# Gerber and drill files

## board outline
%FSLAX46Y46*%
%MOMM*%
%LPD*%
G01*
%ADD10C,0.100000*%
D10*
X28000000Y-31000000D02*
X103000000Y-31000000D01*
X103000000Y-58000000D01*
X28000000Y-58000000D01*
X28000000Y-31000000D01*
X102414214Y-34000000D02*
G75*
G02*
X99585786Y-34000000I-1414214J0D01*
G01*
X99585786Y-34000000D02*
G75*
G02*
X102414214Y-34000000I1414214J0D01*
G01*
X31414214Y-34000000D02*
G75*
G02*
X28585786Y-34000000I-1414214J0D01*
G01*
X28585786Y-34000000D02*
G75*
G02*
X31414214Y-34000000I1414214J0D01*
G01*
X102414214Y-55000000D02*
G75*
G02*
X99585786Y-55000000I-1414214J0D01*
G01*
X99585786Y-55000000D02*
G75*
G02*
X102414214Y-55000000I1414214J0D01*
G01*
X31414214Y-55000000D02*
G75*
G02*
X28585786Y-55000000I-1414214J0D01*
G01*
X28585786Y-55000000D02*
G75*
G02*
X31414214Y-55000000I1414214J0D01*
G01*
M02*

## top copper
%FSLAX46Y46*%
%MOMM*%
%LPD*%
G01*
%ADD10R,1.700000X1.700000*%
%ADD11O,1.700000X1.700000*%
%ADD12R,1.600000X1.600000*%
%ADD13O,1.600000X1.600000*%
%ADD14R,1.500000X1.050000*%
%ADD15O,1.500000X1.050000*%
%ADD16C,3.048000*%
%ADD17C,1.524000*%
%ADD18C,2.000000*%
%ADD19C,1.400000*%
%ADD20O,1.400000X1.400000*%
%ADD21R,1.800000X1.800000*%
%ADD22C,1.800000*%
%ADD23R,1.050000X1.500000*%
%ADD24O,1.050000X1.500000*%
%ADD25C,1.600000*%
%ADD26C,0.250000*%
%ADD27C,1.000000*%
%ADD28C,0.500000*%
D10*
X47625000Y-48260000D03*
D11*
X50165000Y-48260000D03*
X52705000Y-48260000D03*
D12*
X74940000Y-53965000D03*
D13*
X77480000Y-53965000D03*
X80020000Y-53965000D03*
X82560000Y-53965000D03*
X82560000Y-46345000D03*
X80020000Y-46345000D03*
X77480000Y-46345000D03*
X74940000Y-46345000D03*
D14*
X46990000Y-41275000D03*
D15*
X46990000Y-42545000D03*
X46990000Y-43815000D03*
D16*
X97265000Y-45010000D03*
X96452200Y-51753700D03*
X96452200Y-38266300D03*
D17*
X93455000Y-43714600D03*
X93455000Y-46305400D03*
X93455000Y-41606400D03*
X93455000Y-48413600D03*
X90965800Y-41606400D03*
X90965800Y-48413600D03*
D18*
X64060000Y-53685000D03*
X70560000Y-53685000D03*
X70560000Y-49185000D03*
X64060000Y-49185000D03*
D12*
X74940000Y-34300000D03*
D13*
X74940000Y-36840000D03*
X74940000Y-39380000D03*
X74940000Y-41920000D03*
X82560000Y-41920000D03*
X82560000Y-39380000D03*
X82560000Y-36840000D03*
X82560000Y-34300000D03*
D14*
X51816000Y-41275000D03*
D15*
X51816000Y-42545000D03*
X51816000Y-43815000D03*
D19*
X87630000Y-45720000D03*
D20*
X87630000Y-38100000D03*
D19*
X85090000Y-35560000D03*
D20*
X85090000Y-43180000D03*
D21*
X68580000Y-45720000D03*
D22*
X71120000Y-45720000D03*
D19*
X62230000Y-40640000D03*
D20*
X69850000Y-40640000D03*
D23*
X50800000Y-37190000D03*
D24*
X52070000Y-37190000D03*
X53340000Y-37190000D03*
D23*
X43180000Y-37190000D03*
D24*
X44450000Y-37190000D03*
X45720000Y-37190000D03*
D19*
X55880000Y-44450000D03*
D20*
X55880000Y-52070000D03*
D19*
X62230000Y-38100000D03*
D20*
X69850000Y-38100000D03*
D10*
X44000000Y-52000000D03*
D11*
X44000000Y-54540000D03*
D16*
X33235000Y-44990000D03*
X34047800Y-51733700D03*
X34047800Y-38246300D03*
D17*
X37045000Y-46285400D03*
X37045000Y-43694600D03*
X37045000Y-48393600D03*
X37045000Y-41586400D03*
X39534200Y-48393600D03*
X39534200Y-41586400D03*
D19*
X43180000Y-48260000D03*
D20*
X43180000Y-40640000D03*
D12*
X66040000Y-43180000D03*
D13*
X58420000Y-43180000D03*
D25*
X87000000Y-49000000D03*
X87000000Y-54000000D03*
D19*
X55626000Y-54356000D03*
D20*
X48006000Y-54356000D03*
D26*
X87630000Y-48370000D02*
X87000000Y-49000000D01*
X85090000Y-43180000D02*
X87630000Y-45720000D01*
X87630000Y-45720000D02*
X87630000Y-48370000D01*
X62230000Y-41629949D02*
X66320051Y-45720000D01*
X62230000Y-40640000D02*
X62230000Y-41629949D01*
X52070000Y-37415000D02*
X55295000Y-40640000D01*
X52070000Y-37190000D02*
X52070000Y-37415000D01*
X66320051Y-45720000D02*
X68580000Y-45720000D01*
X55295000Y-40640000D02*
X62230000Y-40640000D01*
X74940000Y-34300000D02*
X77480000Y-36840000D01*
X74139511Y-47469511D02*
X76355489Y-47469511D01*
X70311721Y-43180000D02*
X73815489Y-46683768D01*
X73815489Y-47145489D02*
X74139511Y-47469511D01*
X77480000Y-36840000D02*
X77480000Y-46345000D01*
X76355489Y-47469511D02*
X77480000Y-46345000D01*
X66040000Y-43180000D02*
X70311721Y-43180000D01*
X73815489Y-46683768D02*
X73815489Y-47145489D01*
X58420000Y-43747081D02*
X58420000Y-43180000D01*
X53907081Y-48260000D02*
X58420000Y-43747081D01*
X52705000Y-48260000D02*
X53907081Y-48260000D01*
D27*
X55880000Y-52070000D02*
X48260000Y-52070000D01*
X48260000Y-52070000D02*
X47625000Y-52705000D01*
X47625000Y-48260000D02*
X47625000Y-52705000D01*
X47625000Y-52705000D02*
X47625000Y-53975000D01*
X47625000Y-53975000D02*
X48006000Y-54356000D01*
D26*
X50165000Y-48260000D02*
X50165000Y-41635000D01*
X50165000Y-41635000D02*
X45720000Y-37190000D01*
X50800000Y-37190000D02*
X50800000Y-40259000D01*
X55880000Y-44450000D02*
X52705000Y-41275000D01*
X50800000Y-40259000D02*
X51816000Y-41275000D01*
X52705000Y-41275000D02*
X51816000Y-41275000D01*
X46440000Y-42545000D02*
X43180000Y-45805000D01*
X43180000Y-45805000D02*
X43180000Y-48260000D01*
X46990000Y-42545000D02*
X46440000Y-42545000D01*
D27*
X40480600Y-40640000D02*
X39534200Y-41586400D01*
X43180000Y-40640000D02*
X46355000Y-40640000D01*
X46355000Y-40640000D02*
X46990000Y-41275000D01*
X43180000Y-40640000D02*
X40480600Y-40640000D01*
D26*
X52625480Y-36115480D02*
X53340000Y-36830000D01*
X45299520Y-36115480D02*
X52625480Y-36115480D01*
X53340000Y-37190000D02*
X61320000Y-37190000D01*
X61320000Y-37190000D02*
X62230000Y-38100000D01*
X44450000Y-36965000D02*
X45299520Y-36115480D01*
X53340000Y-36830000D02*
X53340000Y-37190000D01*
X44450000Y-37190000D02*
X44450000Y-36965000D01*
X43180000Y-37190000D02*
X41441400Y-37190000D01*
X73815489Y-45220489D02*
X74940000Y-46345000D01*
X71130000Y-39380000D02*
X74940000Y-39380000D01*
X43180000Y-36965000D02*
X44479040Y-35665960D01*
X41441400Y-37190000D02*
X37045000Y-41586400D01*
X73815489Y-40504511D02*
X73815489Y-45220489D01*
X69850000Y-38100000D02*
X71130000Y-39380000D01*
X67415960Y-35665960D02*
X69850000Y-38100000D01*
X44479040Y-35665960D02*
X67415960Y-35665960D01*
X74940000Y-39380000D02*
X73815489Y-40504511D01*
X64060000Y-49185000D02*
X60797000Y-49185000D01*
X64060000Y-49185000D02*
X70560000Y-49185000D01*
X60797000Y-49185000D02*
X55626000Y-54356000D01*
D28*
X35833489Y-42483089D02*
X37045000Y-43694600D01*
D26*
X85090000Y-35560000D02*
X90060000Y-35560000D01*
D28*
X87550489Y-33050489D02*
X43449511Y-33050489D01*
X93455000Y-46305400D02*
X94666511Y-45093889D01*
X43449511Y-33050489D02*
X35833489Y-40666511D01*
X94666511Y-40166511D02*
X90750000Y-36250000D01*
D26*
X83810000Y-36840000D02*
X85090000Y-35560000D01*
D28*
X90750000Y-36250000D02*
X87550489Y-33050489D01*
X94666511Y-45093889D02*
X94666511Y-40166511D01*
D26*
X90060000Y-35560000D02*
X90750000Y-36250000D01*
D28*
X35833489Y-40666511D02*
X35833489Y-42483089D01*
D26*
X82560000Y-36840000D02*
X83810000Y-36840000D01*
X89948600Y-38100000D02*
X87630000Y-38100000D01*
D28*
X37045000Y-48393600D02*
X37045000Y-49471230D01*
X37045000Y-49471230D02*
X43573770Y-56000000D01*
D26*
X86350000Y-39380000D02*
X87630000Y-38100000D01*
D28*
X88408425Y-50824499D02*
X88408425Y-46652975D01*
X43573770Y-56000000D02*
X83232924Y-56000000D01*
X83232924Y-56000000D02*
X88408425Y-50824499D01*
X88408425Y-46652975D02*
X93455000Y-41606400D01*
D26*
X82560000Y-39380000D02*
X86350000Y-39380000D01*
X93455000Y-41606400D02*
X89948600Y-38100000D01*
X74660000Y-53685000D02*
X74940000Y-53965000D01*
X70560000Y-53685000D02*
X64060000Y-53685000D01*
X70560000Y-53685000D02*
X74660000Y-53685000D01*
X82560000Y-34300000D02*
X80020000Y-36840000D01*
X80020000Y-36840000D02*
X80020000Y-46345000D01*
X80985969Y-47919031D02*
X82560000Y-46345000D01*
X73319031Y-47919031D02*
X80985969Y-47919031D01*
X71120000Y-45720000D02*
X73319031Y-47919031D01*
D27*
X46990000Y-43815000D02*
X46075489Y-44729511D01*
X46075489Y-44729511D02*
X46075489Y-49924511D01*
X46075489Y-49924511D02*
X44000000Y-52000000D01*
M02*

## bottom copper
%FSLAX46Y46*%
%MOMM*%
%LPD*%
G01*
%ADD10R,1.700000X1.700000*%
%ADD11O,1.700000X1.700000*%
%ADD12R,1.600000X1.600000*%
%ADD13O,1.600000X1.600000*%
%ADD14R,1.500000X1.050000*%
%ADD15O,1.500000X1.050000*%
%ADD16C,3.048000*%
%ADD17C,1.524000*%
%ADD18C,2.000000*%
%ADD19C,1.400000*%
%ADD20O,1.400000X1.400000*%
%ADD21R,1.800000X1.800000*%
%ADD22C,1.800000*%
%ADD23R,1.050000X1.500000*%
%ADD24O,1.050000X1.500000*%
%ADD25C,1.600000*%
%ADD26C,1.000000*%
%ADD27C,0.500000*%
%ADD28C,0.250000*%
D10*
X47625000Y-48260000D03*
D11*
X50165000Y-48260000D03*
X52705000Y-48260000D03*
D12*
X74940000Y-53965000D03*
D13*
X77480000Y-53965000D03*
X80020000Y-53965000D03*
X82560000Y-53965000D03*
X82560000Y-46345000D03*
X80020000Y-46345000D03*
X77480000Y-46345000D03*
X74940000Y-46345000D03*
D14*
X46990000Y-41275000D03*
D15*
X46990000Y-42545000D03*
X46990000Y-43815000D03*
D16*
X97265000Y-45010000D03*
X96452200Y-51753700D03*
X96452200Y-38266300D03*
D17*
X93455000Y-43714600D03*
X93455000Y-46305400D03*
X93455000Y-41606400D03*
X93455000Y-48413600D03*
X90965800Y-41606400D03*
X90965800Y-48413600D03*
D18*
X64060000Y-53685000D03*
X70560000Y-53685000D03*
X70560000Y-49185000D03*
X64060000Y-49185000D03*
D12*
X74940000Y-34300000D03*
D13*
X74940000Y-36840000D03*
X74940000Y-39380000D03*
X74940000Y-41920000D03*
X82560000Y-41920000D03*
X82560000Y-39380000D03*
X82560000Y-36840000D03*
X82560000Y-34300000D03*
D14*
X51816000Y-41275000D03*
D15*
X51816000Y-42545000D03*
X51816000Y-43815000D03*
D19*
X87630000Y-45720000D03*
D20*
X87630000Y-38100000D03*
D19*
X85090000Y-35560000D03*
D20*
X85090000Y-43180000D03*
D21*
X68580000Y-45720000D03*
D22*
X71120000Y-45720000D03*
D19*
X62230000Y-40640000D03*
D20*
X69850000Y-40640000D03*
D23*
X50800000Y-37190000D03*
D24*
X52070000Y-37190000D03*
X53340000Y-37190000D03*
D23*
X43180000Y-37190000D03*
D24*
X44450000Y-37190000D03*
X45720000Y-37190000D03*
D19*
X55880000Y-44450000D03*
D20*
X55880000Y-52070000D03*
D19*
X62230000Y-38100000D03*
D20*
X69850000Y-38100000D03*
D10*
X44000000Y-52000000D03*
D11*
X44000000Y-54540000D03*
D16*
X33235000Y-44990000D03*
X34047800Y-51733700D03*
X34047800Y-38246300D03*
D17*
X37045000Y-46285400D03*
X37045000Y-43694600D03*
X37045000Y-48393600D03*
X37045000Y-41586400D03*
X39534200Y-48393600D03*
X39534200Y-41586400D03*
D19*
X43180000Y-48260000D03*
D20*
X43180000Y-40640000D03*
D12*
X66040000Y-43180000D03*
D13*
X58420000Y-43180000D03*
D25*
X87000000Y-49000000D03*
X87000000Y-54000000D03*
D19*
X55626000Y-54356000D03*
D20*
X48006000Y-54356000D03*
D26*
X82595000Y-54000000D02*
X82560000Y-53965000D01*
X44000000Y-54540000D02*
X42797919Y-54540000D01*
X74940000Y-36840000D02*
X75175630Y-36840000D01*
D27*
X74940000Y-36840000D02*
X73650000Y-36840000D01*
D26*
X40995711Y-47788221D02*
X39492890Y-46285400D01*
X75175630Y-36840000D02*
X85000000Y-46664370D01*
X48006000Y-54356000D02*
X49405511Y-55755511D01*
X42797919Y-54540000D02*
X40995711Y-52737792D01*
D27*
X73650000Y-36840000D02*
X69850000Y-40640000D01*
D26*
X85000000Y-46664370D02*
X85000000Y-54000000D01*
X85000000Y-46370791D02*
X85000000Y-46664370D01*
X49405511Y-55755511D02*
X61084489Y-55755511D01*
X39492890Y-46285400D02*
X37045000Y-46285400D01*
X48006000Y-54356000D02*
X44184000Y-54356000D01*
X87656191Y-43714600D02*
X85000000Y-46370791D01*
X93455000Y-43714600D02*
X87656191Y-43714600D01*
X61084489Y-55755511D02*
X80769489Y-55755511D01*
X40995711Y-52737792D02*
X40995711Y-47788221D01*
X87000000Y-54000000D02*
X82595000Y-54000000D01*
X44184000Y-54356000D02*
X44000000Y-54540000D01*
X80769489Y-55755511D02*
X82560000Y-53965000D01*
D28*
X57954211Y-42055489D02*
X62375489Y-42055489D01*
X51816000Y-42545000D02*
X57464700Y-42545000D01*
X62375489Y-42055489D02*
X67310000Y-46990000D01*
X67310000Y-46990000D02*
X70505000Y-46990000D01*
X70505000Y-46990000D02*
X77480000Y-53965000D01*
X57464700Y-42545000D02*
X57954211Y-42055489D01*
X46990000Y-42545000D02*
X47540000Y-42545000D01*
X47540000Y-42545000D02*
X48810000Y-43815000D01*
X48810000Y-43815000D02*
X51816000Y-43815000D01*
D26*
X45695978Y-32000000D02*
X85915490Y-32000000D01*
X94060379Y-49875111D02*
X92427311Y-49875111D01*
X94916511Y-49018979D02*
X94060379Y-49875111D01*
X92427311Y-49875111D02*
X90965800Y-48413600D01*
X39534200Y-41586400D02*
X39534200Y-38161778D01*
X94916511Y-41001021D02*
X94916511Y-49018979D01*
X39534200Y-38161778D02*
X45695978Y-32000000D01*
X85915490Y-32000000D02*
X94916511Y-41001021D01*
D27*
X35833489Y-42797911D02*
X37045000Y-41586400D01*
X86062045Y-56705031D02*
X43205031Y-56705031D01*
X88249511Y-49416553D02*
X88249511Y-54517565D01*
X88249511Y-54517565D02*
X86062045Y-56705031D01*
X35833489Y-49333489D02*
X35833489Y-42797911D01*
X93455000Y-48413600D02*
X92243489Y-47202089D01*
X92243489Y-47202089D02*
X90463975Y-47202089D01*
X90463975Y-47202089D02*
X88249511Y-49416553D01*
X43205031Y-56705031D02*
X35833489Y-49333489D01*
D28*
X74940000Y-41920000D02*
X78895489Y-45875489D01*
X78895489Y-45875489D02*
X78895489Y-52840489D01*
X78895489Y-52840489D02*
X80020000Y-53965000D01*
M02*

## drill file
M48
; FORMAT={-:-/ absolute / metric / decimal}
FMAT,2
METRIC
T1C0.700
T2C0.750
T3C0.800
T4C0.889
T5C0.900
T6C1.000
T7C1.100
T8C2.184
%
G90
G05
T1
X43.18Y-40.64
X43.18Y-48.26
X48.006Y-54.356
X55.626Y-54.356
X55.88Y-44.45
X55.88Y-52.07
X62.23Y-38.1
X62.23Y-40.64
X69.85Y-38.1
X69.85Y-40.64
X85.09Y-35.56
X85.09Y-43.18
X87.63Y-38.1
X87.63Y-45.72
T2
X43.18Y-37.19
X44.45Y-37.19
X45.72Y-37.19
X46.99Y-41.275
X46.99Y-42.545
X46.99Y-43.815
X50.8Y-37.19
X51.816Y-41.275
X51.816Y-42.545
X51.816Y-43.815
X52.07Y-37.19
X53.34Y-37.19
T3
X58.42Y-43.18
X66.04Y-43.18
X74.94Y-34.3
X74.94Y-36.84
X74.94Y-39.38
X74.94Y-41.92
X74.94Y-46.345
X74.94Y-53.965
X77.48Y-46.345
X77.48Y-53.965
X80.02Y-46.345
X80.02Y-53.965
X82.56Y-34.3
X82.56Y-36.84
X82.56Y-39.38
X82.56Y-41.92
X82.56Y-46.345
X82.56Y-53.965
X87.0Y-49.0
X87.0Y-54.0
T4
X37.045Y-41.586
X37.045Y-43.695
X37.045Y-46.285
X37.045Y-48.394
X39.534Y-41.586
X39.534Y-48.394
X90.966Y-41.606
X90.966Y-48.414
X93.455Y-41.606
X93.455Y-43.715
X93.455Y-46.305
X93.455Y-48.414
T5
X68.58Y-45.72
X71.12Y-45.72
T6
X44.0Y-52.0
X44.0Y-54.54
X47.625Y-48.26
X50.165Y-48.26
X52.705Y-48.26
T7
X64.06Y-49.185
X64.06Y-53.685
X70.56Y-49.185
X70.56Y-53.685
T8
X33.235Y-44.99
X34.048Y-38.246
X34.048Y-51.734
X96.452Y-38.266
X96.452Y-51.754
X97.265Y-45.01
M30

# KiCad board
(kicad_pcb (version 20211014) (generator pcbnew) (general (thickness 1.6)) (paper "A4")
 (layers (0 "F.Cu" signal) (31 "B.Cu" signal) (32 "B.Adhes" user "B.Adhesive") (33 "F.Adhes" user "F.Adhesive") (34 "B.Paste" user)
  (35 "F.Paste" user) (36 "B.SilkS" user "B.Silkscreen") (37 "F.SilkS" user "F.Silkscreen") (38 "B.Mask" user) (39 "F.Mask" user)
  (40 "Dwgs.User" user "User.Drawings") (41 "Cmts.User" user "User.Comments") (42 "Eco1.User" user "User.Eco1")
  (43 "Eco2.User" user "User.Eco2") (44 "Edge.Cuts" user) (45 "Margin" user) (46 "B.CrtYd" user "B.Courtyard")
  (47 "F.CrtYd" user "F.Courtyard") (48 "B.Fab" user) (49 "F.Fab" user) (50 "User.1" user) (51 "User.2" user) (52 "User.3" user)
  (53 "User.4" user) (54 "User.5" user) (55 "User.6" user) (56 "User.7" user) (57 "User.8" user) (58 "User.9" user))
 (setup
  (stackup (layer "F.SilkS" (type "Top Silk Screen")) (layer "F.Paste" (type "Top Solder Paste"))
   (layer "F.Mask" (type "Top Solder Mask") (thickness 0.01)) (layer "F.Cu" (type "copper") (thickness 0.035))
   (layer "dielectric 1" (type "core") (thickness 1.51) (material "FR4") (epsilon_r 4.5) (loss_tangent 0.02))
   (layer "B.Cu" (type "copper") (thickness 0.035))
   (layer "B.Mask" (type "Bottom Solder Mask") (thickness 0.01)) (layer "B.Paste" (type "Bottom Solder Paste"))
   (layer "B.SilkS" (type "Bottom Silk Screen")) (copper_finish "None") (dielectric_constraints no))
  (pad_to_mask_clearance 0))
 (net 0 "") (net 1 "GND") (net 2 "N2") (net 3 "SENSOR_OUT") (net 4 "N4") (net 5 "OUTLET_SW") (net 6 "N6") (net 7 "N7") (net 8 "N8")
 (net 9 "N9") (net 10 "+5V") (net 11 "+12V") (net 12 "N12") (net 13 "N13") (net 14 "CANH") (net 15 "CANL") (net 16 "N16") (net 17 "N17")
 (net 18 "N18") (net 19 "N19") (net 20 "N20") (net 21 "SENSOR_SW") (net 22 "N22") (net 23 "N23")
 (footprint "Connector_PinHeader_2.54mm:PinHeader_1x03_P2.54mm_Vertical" (layer "F.Cu") (at 47.625 48.26 90)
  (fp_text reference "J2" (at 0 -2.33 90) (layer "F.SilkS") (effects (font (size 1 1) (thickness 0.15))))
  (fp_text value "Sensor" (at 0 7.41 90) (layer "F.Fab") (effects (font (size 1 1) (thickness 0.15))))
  (pad "1" thru_hole rect (at 0 0 90) (size 1.7 1.7) (drill 1) (layers *.Cu *.Mask) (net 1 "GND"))
  (pad "2" thru_hole oval (at 0 2.54 90) (size 1.7 1.7) (drill 1) (layers *.Cu *.Mask) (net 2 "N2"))
  (pad "3" thru_hole oval (at 0 5.08 90) (size 1.7 1.7) (drill 1) (layers *.Cu *.Mask) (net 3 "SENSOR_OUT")))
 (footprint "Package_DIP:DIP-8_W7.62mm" (layer "F.Cu") (at 74.94 53.965 90)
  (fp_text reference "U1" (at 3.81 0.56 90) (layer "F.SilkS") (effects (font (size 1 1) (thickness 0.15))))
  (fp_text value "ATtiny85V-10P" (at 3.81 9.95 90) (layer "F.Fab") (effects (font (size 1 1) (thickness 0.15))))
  (pad "1" thru_hole rect (at 0 0 90) (size 1.6 1.6) (drill 0.8) (layers *.Cu *.Mask) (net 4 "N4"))
  (pad "2" thru_hole oval (at 0 2.54 90) (size 1.6 1.6) (drill 0.8) (layers *.Cu *.Mask) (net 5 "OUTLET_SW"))
  (pad "3" thru_hole oval (at 0 5.08 90) (size 1.6 1.6) (drill 0.8) (layers *.Cu *.Mask) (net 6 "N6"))
  (pad "4" thru_hole oval (at 0 7.62 90) (size 1.6 1.6) (drill 0.8) (layers *.Cu *.Mask) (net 1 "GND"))
  (pad "5" thru_hole oval (at 7.62 7.62 90) (size 1.6 1.6) (drill 0.8) (layers *.Cu *.Mask) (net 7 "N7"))
  (pad "6" thru_hole oval (at 7.62 5.08 90) (size 1.6 1.6) (drill 0.8) (layers *.Cu *.Mask) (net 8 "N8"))
  (pad "7" thru_hole oval (at 7.62 2.54 90) (size 1.6 1.6) (drill 0.8) (layers *.Cu *.Mask) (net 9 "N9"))
  (pad "8" thru_hole oval (at 7.62 0 90) (size 1.6 1.6) (drill 0.8) (layers *.Cu *.Mask) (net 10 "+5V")))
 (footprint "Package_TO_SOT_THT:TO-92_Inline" (layer "F.Cu") (at 46.99 41.275 -90)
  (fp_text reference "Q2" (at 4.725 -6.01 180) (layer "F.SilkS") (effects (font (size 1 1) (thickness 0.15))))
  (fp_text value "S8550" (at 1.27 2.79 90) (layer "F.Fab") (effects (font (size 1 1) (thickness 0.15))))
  (pad "1" thru_hole rect (at 0 0 270) (size 1.05 1.5) (drill 0.75) (layers *.Cu *.Mask) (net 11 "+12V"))
  (pad "2" thru_hole oval (at 1.27 0 270) (size 1.05 1.5) (drill 0.75) (layers *.Cu *.Mask) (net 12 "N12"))
  (pad "3" thru_hole oval (at 2.54 0 270) (size 1.05 1.5) (drill 0.75) (layers *.Cu *.Mask) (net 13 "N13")))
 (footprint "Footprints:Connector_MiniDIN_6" (layer "F.Cu") (at 97.265 45.01 -90)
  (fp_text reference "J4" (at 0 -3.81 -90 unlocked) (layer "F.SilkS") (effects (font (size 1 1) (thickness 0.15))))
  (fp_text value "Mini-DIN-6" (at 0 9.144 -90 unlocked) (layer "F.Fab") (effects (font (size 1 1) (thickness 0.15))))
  (pad "" thru_hole circle (at 0 0 270) (size 3.048 3.048) (drill 2.1844) (layers *.Cu *.Mask))
  (pad "" thru_hole circle (at 6.7437 0.8128 270) (size 3.048 3.048) (drill 2.1844) (layers *.Cu *.Mask))
  (pad "" thru_hole circle (at -6.7437 0.8128 270) (size 3.048 3.048) (drill 2.1844) (layers *.Cu *.Mask))
  (pad "1" thru_hole circle (at -1.2954 3.81 270) (size 1.524 1.524) (drill 0.889) (layers *.Cu *.Mask) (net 1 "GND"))
  (pad "2" thru_hole circle (at 1.2954 3.81 270) (size 1.524 1.524) (drill 0.889) (layers *.Cu *.Mask) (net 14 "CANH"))
  (pad "3" thru_hole circle (at -3.4036 3.81 270) (size 1.524 1.524) (drill 0.889) (layers *.Cu *.Mask) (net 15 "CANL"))
  (pad "4" thru_hole circle (at 3.4036 3.81 270) (size 1.524 1.524) (drill 0.889) (layers *.Cu *.Mask) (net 10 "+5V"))
  (pad "5" thru_hole circle (at -3.4036 6.2992 270) (size 1.524 1.524) (drill 0.889) (layers *.Cu *.Mask) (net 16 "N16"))
  (pad "6" thru_hole circle (at 3.4036 6.2992 270) (size 1.524 1.524) (drill 0.889) (layers *.Cu *.Mask) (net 11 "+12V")))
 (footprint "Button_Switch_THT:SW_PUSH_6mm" (layer "F.Cu") (at 70.56 53.685 180)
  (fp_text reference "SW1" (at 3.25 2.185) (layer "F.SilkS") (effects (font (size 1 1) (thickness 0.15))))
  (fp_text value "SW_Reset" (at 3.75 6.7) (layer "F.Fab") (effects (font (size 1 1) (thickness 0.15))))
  (pad "1" thru_hole circle (at 6.5 0 270) (size 2 2) (drill 1.1) (layers *.Cu *.Mask) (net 4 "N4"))
  (pad "1" thru_hole circle (at 0 0 270) (size 2 2) (drill 1.1) (layers *.Cu *.Mask) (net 4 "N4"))
  (pad "2" thru_hole circle (at 0 4.5 270) (size 2 2) (drill 1.1) (layers *.Cu *.Mask) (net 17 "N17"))
  (pad "2" thru_hole circle (at 6.5 4.5 270) (size 2 2) (drill 1.1) (layers *.Cu *.Mask) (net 17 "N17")))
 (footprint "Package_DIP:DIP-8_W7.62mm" (layer "F.Cu") (at 74.94 34.3)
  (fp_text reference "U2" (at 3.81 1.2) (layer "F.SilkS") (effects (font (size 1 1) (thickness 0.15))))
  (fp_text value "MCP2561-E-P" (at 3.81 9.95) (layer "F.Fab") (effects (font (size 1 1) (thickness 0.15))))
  (pad "1" thru_hole rect (at 0 0) (size 1.6 1.6) (drill 0.8) (layers *.Cu *.Mask) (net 9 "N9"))
  (pad "2" thru_hole oval (at 0 2.54) (size 1.6 1.6) (drill 0.8) (layers *.Cu *.Mask) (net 1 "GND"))
  (pad "3" thru_hole oval (at 0 5.08) (size 1.6 1.6) (drill 0.8) (layers *.Cu *.Mask) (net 10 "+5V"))
  (pad "4" thru_hole oval (at 0 7.62) (size 1.6 1.6) (drill 0.8) (layers *.Cu *.Mask) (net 6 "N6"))
  (pad "5" thru_hole oval (at 7.62 7.62) (size 1.6 1.6) (drill 0.8) (layers *.Cu *.Mask) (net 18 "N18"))
  (pad "6" thru_hole oval (at 7.62 5.08) (size 1.6 1.6) (drill 0.8) (layers *.Cu *.Mask) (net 15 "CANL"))
  (pad "7" thru_hole oval (at 7.62 2.54) (size 1.6 1.6) (drill 0.8) (layers *.Cu *.Mask) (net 14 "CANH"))
  (pad "8" thru_hole oval (at 7.62 0) (size 1.6 1.6) (drill 0.8) (layers *.Cu *.Mask) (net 8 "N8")))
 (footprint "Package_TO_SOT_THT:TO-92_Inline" (layer "F.Cu") (at 51.816 41.275 -90)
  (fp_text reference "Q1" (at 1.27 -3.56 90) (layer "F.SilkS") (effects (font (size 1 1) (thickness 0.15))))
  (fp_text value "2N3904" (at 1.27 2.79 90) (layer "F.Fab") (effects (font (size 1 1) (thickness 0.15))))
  (pad "1" thru_hole rect (at 0 0 270) (size 1.05 1.5) (drill 0.75) (layers *.Cu *.Mask) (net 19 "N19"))
  (pad "2" thru_hole oval (at 1.27 0 270) (size 1.05 1.5) (drill 0.75) (layers *.Cu *.Mask) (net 5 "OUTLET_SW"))
  (pad "3" thru_hole oval (at 2.54 0 270) (size 1.05 1.5) (drill 0.75) (layers *.Cu *.Mask) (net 12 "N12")))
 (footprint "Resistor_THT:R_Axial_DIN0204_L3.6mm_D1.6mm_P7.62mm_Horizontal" (layer "F.Cu") (at 87.63 45.72 90)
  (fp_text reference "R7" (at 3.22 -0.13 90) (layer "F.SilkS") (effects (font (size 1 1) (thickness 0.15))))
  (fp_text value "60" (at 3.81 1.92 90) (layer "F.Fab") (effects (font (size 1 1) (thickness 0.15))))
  (pad "1" thru_hole circle (at 0 0 90) (size 1.4 1.4) (drill 0.7) (layers *.Cu *.Mask) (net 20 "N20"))
  (pad "2" thru_hole oval (at 7.62 0 90) (size 1.4 1.4) (drill 0.7) (layers *.Cu *.Mask) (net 15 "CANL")))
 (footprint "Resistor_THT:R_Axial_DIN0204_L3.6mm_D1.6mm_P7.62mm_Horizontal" (layer "F.Cu") (at 85.09 35.56 -90)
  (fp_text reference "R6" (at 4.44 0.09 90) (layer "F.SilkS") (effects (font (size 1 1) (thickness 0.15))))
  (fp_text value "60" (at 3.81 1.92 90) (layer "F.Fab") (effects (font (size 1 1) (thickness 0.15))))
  (pad "1" thru_hole circle (at 0 0 270) (size 1.4 1.4) (drill 0.7) (layers *.Cu *.Mask) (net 14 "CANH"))
  (pad "2" thru_hole oval (at 7.62 0 270) (size 1.4 1.4) (drill 0.7) (layers *.Cu *.Mask) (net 20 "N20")))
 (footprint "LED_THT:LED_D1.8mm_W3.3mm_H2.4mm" (layer "F.Cu") (at 68.58 45.72)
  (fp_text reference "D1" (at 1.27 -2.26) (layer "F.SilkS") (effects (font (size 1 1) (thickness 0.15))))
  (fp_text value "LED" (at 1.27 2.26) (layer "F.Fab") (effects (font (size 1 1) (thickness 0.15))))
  (pad "1" thru_hole rect (at 0 0) (size 1.8 1.8) (drill 0.9) (layers *.Cu *.Mask) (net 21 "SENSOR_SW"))
  (pad "2" thru_hole circle (at 2.54 0) (size 1.8 1.8) (drill 0.9) (layers *.Cu *.Mask) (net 7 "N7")))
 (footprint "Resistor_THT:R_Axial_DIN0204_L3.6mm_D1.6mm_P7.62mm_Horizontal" (layer "F.Cu") (at 62.23 40.64)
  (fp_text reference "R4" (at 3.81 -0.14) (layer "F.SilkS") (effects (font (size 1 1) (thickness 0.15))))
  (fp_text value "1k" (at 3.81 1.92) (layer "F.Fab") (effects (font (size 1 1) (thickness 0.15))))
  (pad "1" thru_hole circle (at 0 0) (size 1.4 1.4) (drill 0.7) (layers *.Cu *.Mask) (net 21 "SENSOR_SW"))
  (pad "2" thru_hole oval (at 7.62 0) (size 1.4 1.4) (drill 0.7) (layers *.Cu *.Mask) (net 1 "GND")))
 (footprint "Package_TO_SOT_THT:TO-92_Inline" (layer "F.Cu") (at 50.8 37.19)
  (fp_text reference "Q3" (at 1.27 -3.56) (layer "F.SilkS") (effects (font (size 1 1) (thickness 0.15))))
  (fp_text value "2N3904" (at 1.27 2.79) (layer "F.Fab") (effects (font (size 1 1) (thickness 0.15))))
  (pad "1" thru_hole rect (at 0 0) (size 1.05 1.5) (drill 0.75) (layers *.Cu *.Mask) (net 19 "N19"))
  (pad "2" thru_hole oval (at 1.27 0) (size 1.05 1.5) (drill 0.75) (layers *.Cu *.Mask) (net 21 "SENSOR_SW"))
  (pad "3" thru_hole oval (at 2.54 0) (size 1.05 1.5) (drill 0.75) (layers *.Cu *.Mask) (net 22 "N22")))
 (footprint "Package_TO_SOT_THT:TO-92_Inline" (layer "F.Cu") (at 43.18 37.19)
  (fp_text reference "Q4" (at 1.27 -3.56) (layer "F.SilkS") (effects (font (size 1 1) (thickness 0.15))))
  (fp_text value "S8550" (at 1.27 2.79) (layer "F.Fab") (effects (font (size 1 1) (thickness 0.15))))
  (pad "1" thru_hole rect (at 0 0) (size 1.05 1.5) (drill 0.75) (layers *.Cu *.Mask) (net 10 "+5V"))
  (pad "2" thru_hole oval (at 1.27 0) (size 1.05 1.5) (drill 0.75) (layers *.Cu *.Mask) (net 22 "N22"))
  (pad "3" thru_hole oval (at 2.54 0) (size 1.05 1.5) (drill 0.75) (layers *.Cu *.Mask) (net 2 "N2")))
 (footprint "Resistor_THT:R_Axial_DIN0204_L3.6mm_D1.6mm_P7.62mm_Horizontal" (layer "F.Cu") (at 55.88 44.45 -90)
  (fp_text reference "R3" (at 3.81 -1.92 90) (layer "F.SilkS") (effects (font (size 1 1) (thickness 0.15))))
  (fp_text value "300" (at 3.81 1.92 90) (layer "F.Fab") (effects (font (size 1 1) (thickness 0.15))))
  (pad "1" thru_hole circle (at 0 0 270) (size 1.4 1.4) (drill 0.7) (layers *.Cu *.Mask) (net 19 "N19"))
  (pad "2" thru_hole oval (at 7.62 0 270) (size 1.4 1.4) (drill 0.7) (layers *.Cu *.Mask) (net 1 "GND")))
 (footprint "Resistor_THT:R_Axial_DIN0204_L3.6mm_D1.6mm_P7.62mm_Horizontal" (layer "F.Cu") (at 62.23 38.1)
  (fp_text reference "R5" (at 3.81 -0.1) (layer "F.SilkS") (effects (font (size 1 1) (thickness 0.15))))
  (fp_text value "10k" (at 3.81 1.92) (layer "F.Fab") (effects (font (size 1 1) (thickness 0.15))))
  (pad "1" thru_hole circle (at 0 0) (size 1.4 1.4) (drill 0.7) (layers *.Cu *.Mask) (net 22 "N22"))
  (pad "2" thru_hole oval (at 7.62 0) (size 1.4 1.4) (drill 0.7) (layers *.Cu *.Mask) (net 10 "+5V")))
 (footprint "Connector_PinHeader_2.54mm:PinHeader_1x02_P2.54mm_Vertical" (layer "F.Cu") (at 44 52)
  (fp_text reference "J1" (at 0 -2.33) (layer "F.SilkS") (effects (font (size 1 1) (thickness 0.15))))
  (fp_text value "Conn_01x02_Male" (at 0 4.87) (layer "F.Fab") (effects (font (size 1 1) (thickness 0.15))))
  (pad "1" thru_hole rect (at 0 0) (size 1.7 1.7) (drill 1) (layers *.Cu *.Mask) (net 13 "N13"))
  (pad "2" thru_hole oval (at 0 2.54) (size 1.7 1.7) (drill 1) (layers *.Cu *.Mask) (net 1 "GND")))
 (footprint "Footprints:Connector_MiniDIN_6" (layer "F.Cu") (at 33.235 44.99 90)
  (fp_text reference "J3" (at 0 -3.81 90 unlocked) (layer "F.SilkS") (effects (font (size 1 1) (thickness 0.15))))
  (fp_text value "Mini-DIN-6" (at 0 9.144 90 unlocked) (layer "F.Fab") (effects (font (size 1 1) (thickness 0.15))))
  (pad "" thru_hole circle (at 0 0 90) (size 3.048 3.048) (drill 2.1844) (layers *.Cu *.Mask))
  (pad "" thru_hole circle (at -6.7437 0.8128 90) (size 3.048 3.048) (drill 2.1844) (layers *.Cu *.Mask))
  (pad "" thru_hole circle (at 6.7437 0.8128 90) (size 3.048 3.048) (drill 2.1844) (layers *.Cu *.Mask))
  (pad "1" thru_hole circle (at -1.2954 3.81 90) (size 1.524 1.524) (drill 0.889) (layers *.Cu *.Mask) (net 1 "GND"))
  (pad "2" thru_hole circle (at 1.2954 3.81 90) (size 1.524 1.524) (drill 0.889) (layers *.Cu *.Mask) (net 14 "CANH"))
  (pad "3" thru_hole circle (at -3.4036 3.81 90) (size 1.524 1.524) (drill 0.889) (layers *.Cu *.Mask) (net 15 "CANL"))
  (pad "4" thru_hole circle (at 3.4036 3.81 90) (size 1.524 1.524) (drill 0.889) (layers *.Cu *.Mask) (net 10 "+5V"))
  (pad "5" thru_hole circle (at -3.4036 6.2992 90) (size 1.524 1.524) (drill 0.889) (layers *.Cu *.Mask) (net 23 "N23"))
  (pad "6" thru_hole circle (at 3.4036 6.2992 90) (size 1.524 1.524) (drill 0.889) (layers *.Cu *.Mask) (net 11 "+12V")))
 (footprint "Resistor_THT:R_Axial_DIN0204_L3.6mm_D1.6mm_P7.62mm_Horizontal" (layer "F.Cu") (at 43.18 48.26 90)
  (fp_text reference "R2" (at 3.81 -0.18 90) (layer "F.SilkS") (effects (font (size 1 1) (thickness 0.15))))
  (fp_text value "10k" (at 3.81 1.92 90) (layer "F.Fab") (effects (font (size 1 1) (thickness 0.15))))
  (pad "1" thru_hole circle (at 0 0 90) (size 1.4 1.4) (drill 0.7) (layers *.Cu *.Mask) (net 12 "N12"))
  (pad "2" thru_hole oval (at 7.62 0 90) (size 1.4 1.4) (drill 0.7) (layers *.Cu *.Mask) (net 11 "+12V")))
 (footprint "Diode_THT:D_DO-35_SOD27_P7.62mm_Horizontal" (layer "F.Cu") (at 66.04 43.18 180)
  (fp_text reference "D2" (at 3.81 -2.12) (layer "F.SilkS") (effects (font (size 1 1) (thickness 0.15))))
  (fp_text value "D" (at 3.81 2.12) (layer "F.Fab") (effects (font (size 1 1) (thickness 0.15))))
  (pad "1" thru_hole rect (at 0 0 180) (size 1.6 1.6) (drill 0.8) (layers *.Cu *.Mask) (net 9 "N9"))
  (pad "2" thru_hole oval (at 7.62 0 180) (size 1.6 1.6) (drill 0.8) (layers *.Cu *.Mask) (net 3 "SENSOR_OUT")))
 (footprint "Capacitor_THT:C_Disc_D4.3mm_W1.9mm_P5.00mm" (layer "F.Cu") (at 87 49 -90)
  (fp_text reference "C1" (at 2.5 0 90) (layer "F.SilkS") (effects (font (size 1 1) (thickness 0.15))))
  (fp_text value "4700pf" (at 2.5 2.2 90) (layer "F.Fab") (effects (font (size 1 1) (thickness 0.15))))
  (pad "1" thru_hole circle (at 0 0 270) (size 1.6 1.6) (drill 0.8) (layers *.Cu *.Mask) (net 20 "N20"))
  (pad "2" thru_hole circle (at 5 0 270) (size 1.6 1.6) (drill 0.8) (layers *.Cu *.Mask) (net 1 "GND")))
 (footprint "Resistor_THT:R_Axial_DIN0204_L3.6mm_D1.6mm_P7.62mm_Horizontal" (layer "F.Cu") (at 55.626 54.356 180)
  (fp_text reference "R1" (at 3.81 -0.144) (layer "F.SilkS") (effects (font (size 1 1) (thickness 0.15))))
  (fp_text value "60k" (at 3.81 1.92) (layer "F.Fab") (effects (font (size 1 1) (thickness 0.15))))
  (pad "1" thru_hole circle (at 0 0 180) (size 1.4 1.4) (drill 0.7) (layers *.Cu *.Mask) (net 17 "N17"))
  (pad "2" thru_hole oval (at 7.62 0 180) (size 1.4 1.4) (drill 0.7) (layers *.Cu *.Mask) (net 1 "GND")))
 (gr_rect (start 28 31) (end 103 58) (layer "Edge.Cuts") (width 0.1) (fill none))
 (gr_circle (center 101 34) (end 102 35) (layer "Edge.Cuts") (width 0.1) (fill none))
 (gr_circle (center 30 34) (end 31 35) (layer "Edge.Cuts") (width 0.1) (fill none))
 (gr_circle (center 101 55) (end 102 56) (layer "Edge.Cuts") (width 0.1) (fill none))
 (gr_circle (center 30 55) (end 31 56) (layer "Edge.Cuts") (width 0.1) (fill none))
 (segment (start 87.63 48.37) (end 87 49) (width 0.25) (layer "F.Cu") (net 20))
 (segment (start 85.09 43.18) (end 87.63 45.72) (width 0.25) (layer "F.Cu") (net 20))
 (segment (start 87.63 45.72) (end 87.63 48.37) (width 0.25) (layer "F.Cu") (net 20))
 (segment (start 62.23 41.629949) (end 66.320051 45.72) (width 0.25) (layer "F.Cu") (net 21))
 (segment (start 62.23 40.64) (end 62.23 41.629949) (width 0.25) (layer "F.Cu") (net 21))
 (segment (start 52.07 37.415) (end 55.295 40.64) (width 0.25) (layer "F.Cu") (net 21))
 (segment (start 52.07 37.19) (end 52.07 37.415) (width 0.25) (layer "F.Cu") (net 21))
 (segment (start 66.320051 45.72) (end 68.58 45.72) (width 0.25) (layer "F.Cu") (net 21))
 (segment (start 55.295 40.64) (end 62.23 40.64) (width 0.25) (layer "F.Cu") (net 21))
 (segment (start 74.94 34.3) (end 77.48 36.84) (width 0.25) (layer "F.Cu") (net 9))
 (segment (start 74.139511 47.469511) (end 76.355489 47.469511) (width 0.25) (layer "F.Cu") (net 9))
 (segment (start 70.311721 43.18) (end 73.815489 46.683768) (width 0.25) (layer "F.Cu") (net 9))
 (segment (start 73.815489 47.145489) (end 74.139511 47.469511) (width 0.25) (layer "F.Cu") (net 9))
 (segment (start 77.48 36.84) (end 77.48 46.345) (width 0.25) (layer "F.Cu") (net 9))
 (segment (start 76.355489 47.469511) (end 77.48 46.345) (width 0.25) (layer "F.Cu") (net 9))
 (segment (start 66.04 43.18) (end 70.311721 43.18) (width 0.25) (layer "F.Cu") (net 9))
 (segment (start 73.815489 46.683768) (end 73.815489 47.145489) (width 0.25) (layer "F.Cu") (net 9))
 (segment (start 58.42 43.747081) (end 58.42 43.18) (width 0.25) (layer "F.Cu") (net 3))
 (segment (start 53.907081 48.26) (end 58.42 43.747081) (width 0.25) (layer "F.Cu") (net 3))
 (segment (start 52.705 48.26) (end 53.907081 48.26) (width 0.25) (layer "F.Cu") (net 3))
 (segment (start 55.88 52.07) (end 48.26 52.07) (width 1) (layer "F.Cu") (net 1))
 (segment (start 48.26 52.07) (end 47.625 52.705) (width 1) (layer "F.Cu") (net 1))
 (segment (start 47.625 48.26) (end 47.625 52.705) (width 1) (layer "F.Cu") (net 1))
 (segment (start 47.625 52.705) (end 47.625 53.975) (width 1) (layer "F.Cu") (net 1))
 (segment (start 47.625 53.975) (end 48.006 54.356) (width 1) (layer "F.Cu") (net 1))
 (segment (start 82.595 54) (end 82.56 53.965) (width 1) (layer "B.Cu") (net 1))
 (segment (start 44 54.54) (end 42.797919 54.54) (width 1) (layer "B.Cu") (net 1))
 (segment (start 74.94 36.84) (end 75.17563 36.84) (width 1) (layer "B.Cu") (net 1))
 (segment (start 74.94 36.84) (end 73.65 36.84) (width 0.5) (layer "B.Cu") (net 1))
 (segment (start 40.995711 47.788221) (end 39.49289 46.2854) (width 1) (layer "B.Cu") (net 1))
 (segment (start 75.17563 36.84) (end 85 46.66437) (width 1) (layer "B.Cu") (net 1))
 (segment (start 48.006 54.356) (end 49.405511 55.755511) (width 1) (layer "B.Cu") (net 1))
 (segment (start 42.797919 54.54) (end 40.995711 52.737792) (width 1) (layer "B.Cu") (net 1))
 (segment (start 73.65 36.84) (end 69.85 40.64) (width 0.5) (layer "B.Cu") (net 1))
 (segment (start 85 46.66437) (end 85 54) (width 1) (layer "B.Cu") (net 1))
 (segment (start 85 46.370791) (end 85 46.66437) (width 1) (layer "B.Cu") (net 1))
 (segment (start 49.405511 55.755511) (end 61.084489 55.755511) (width 1) (layer "B.Cu") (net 1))
 (segment (start 39.49289 46.2854) (end 37.045 46.2854) (width 1) (layer "B.Cu") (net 1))
 (segment (start 48.006 54.356) (end 44.184 54.356) (width 1) (layer "B.Cu") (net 1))
 (segment (start 87.656191 43.7146) (end 85 46.370791) (width 1) (layer "B.Cu") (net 1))
 (segment (start 93.455 43.7146) (end 87.656191 43.7146) (width 1) (layer "B.Cu") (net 1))
 (segment (start 61.084489 55.755511) (end 80.769489 55.755511) (width 1) (layer "B.Cu") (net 1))
 (segment (start 40.995711 52.737792) (end 40.995711 47.788221) (width 1) (layer "B.Cu") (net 1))
 (segment (start 87 54) (end 82.595 54) (width 1) (layer "B.Cu") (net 1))
 (segment (start 44.184 54.356) (end 44 54.54) (width 1) (layer "B.Cu") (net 1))
 (segment (start 80.769489 55.755511) (end 82.56 53.965) (width 1) (layer "B.Cu") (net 1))
 (segment (start 50.165 48.26) (end 50.165 41.635) (width 0.25) (layer "F.Cu") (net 2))
 (segment (start 50.165 41.635) (end 45.72 37.19) (width 0.25) (layer "F.Cu") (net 2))
 (segment (start 50.8 37.19) (end 50.8 40.259) (width 0.25) (layer "F.Cu") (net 19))
 (segment (start 55.88 44.45) (end 52.705 41.275) (width 0.25) (layer "F.Cu") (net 19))
 (segment (start 50.8 40.259) (end 51.816 41.275) (width 0.25) (layer "F.Cu") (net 19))
 (segment (start 52.705 41.275) (end 51.816 41.275) (width 0.25) (layer "F.Cu") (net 19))
 (segment (start 57.954211 42.055489) (end 62.375489 42.055489) (width 0.25) (layer "B.Cu") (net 5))
 (segment (start 51.816 42.545) (end 57.4647 42.545) (width 0.25) (layer "B.Cu") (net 5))
 (segment (start 62.375489 42.055489) (end 67.31 46.99) (width 0.25) (layer "B.Cu") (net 5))
 (segment (start 67.31 46.99) (end 70.505 46.99) (width 0.25) (layer "B.Cu") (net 5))
 (segment (start 70.505 46.99) (end 77.48 53.965) (width 0.25) (layer "B.Cu") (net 5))
 (segment (start 57.4647 42.545) (end 57.954211 42.055489) (width 0.25) (layer "B.Cu") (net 5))
 (segment (start 46.44 42.545) (end 43.18 45.805) (width 0.25) (layer "F.Cu") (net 12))
 (segment (start 43.18 45.805) (end 43.18 48.26) (width 0.25) (layer "F.Cu") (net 12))
 (segment (start 46.99 42.545) (end 46.44 42.545) (width 0.25) (layer "F.Cu") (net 12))
 (segment (start 46.99 42.545) (end 47.54 42.545) (width 0.25) (layer "B.Cu") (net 12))
 (segment (start 47.54 42.545) (end 48.81 43.815) (width 0.25) (layer "B.Cu") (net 12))
 (segment (start 48.81 43.815) (end 51.816 43.815) (width 0.25) (layer "B.Cu") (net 12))
 (segment (start 40.4806 40.64) (end 39.5342 41.5864) (width 1) (layer "F.Cu") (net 11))
 (segment (start 43.18 40.64) (end 46.355 40.64) (width 1) (layer "F.Cu") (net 11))
 (segment (start 46.355 40.64) (end 46.99 41.275) (width 1) (layer "F.Cu") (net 11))
 (segment (start 43.18 40.64) (end 40.4806 40.64) (width 1) (layer "F.Cu") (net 11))
 (segment (start 45.695978 32) (end 85.91549 32) (width 1) (layer "B.Cu") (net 11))
 (segment (start 94.060379 49.875111) (end 92.427311 49.875111) (width 1) (layer "B.Cu") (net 11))
 (segment (start 94.916511 49.018979) (end 94.060379 49.875111) (width 1) (layer "B.Cu") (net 11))
 (segment (start 92.427311 49.875111) (end 90.9658 48.4136) (width 1) (layer "B.Cu") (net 11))
 (segment (start 39.5342 41.5864) (end 39.5342 38.161778) (width 1) (layer "B.Cu") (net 11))
 (segment (start 94.916511 41.001021) (end 94.916511 49.018979) (width 1) (layer "B.Cu") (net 11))
 (segment (start 39.5342 38.161778) (end 45.695978 32) (width 1) (layer "B.Cu") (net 11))
 (segment (start 85.91549 32) (end 94.916511 41.001021) (width 1) (layer "B.Cu") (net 11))
 (segment (start 52.62548 36.11548) (end 53.34 36.83) (width 0.25) (layer "F.Cu") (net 22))
 (segment (start 45.29952 36.11548) (end 52.62548 36.11548) (width 0.25) (layer "F.Cu") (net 22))
 (segment (start 53.34 37.19) (end 61.32 37.19) (width 0.25) (layer "F.Cu") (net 22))
 (segment (start 61.32 37.19) (end 62.23 38.1) (width 0.25) (layer "F.Cu") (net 22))
 (segment (start 44.45 36.965) (end 45.29952 36.11548) (width 0.25) (layer "F.Cu") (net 22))
 (segment (start 53.34 36.83) (end 53.34 37.19) (width 0.25) (layer "F.Cu") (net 22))
 (segment (start 44.45 37.19) (end 44.45 36.965) (width 0.25) (layer "F.Cu") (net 22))
 (segment (start 43.18 37.19) (end 41.4414 37.19) (width 0.25) (layer "F.Cu") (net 10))
 (segment (start 73.815489 45.220489) (end 74.94 46.345) (width 0.25) (layer "F.Cu") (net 10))
 (segment (start 71.13 39.38) (end 74.94 39.38) (width 0.25) (layer "F.Cu") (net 10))
 (segment (start 43.18 36.965) (end 44.47904 35.66596) (width 0.25) (layer "F.Cu") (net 10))
 (segment (start 41.4414 37.19) (end 37.045 41.5864) (width 0.25) (layer "F.Cu") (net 10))
 (segment (start 73.815489 40.504511) (end 73.815489 45.220489) (width 0.25) (layer "F.Cu") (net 10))
 (segment (start 69.85 38.1) (end 71.13 39.38) (width 0.25) (layer "F.Cu") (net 10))
 (segment (start 67.41596 35.66596) (end 69.85 38.1) (width 0.25) (layer "F.Cu") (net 10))
 (segment (start 44.47904 35.66596) (end 67.41596 35.66596) (width 0.25) (layer "F.Cu") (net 10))
 (segment (start 74.94 39.38) (end 73.815489 40.504511) (width 0.25) (layer "F.Cu") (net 10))
 (segment (start 35.833489 42.797911) (end 37.045 41.5864) (width 0.5) (layer "B.Cu") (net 10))
 (segment (start 86.062045 56.705031) (end 43.205031 56.705031) (width 0.5) (layer "B.Cu") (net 10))
 (segment (start 88.249511 49.416553) (end 88.249511 54.517565) (width 0.5) (layer "B.Cu") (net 10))
 (segment (start 88.249511 54.517565) (end 86.062045 56.705031) (width 0.5) (layer "B.Cu") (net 10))
 (segment (start 35.833489 49.333489) (end 35.833489 42.797911) (width 0.5) (layer "B.Cu") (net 10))
 (segment (start 93.455 48.4136) (end 92.243489 47.202089) (width 0.5) (layer "B.Cu") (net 10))
 (segment (start 92.243489 47.202089) (end 90.463975 47.202089) (width 0.5) (layer "B.Cu") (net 10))
 (segment (start 90.463975 47.202089) (end 88.249511 49.416553) (width 0.5) (layer "B.Cu") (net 10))
 (segment (start 43.205031 56.705031) (end 35.833489 49.333489) (width 0.5) (layer "B.Cu") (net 10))
 (segment (start 64.06 49.185) (end 60.797 49.185) (width 0.25) (layer "F.Cu") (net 17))
 (segment (start 64.06 49.185) (end 70.56 49.185) (width 0.25) (layer "F.Cu") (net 17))
 (segment (start 60.797 49.185) (end 55.626 54.356) (width 0.25) (layer "F.Cu") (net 17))
 (segment (start 35.833489 42.483089) (end 37.045 43.6946) (width 0.5) (layer "F.Cu") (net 14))
 (segment (start 85.09 35.56) (end 90.06 35.56) (width 0.25) (layer "F.Cu") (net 14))
 (segment (start 87.550489 33.050489) (end 43.449511 33.050489) (width 0.5) (layer "F.Cu") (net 14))
 (segment (start 93.455 46.3054) (end 94.666511 45.093889) (width 0.5) (layer "F.Cu") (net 14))
 (segment (start 43.449511 33.050489) (end 35.833489 40.666511) (width 0.5) (layer "F.Cu") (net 14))
 (segment (start 94.666511 40.166511) (end 90.75 36.25) (width 0.5) (layer "F.Cu") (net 14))
 (segment (start 83.81 36.84) (end 85.09 35.56) (width 0.25) (layer "F.Cu") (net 14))
 (segment (start 90.75 36.25) (end 87.550489 33.050489) (width 0.5) (layer "F.Cu") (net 14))
 (segment (start 94.666511 45.093889) (end 94.666511 40.166511) (width 0.5) (layer "F.Cu") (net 14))
 (segment (start 90.06 35.56) (end 90.75 36.25) (width 0.25) (layer "F.Cu") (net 14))
 (segment (start 35.833489 40.666511) (end 35.833489 42.483089) (width 0.5) (layer "F.Cu") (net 14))
 (segment (start 82.56 36.84) (end 83.81 36.84) (width 0.25) (layer "F.Cu") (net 14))
 (segment (start 89.9486 38.1) (end 87.63 38.1) (width 0.25) (layer "F.Cu") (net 15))
 (segment (start 37.045 48.3936) (end 37.045 49.47123) (width 0.5) (layer "F.Cu") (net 15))
 (segment (start 37.045 49.47123) (end 43.57377 56) (width 0.5) (layer "F.Cu") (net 15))
 (segment (start 86.35 39.38) (end 87.63 38.1) (width 0.25) (layer "F.Cu") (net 15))
 (segment (start 88.408425 50.824499) (end 88.408425 46.652975) (width 0.5) (layer "F.Cu") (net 15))
 (segment (start 43.57377 56) (end 83.232924 56) (width 0.5) (layer "F.Cu") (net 15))
 (segment (start 83.232924 56) (end 88.408425 50.824499) (width 0.5) (layer "F.Cu") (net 15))
 (segment (start 88.408425 46.652975) (end 93.455 41.6064) (width 0.5) (layer "F.Cu") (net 15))
 (segment (start 82.56 39.38) (end 86.35 39.38) (width 0.25) (layer "F.Cu") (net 15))
 (segment (start 93.455 41.6064) (end 89.9486 38.1) (width 0.25) (layer "F.Cu") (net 15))
 (segment (start 74.66 53.685) (end 74.94 53.965) (width 0.25) (layer "F.Cu") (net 4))
 (segment (start 70.56 53.685) (end 64.06 53.685) (width 0.25) (layer "F.Cu") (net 4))
 (segment (start 70.56 53.685) (end 74.66 53.685) (width 0.25) (layer "F.Cu") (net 4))
 (segment (start 74.94 41.92) (end 78.895489 45.875489) (width 0.25) (layer "B.Cu") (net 6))
 (segment (start 78.895489 45.875489) (end 78.895489 52.840489) (width 0.25) (layer "B.Cu") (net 6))
 (segment (start 78.895489 52.840489) (end 80.02 53.965) (width 0.25) (layer "B.Cu") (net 6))
 (segment (start 82.56 34.3) (end 80.02 36.84) (width 0.25) (layer "F.Cu") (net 8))
 (segment (start 80.02 36.84) (end 80.02 46.345) (width 0.25) (layer "F.Cu") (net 8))
 (segment (start 80.985969 47.919031) (end 82.56 46.345) (width 0.25) (layer "F.Cu") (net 7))
 (segment (start 73.319031 47.919031) (end 80.985969 47.919031) (width 0.25) (layer "F.Cu") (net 7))
 (segment (start 71.12 45.72) (end 73.319031 47.919031) (width 0.25) (layer "F.Cu") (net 7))
 (segment (start 46.99 43.815) (end 46.075489 44.729511) (width 1) (layer "F.Cu") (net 13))
 (segment (start 46.075489 44.729511) (end 46.075489 49.924511) (width 1) (layer "F.Cu") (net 13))
 (segment (start 46.075489 49.924511) (end 44 52) (width 1) (layer "F.Cu") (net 13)))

